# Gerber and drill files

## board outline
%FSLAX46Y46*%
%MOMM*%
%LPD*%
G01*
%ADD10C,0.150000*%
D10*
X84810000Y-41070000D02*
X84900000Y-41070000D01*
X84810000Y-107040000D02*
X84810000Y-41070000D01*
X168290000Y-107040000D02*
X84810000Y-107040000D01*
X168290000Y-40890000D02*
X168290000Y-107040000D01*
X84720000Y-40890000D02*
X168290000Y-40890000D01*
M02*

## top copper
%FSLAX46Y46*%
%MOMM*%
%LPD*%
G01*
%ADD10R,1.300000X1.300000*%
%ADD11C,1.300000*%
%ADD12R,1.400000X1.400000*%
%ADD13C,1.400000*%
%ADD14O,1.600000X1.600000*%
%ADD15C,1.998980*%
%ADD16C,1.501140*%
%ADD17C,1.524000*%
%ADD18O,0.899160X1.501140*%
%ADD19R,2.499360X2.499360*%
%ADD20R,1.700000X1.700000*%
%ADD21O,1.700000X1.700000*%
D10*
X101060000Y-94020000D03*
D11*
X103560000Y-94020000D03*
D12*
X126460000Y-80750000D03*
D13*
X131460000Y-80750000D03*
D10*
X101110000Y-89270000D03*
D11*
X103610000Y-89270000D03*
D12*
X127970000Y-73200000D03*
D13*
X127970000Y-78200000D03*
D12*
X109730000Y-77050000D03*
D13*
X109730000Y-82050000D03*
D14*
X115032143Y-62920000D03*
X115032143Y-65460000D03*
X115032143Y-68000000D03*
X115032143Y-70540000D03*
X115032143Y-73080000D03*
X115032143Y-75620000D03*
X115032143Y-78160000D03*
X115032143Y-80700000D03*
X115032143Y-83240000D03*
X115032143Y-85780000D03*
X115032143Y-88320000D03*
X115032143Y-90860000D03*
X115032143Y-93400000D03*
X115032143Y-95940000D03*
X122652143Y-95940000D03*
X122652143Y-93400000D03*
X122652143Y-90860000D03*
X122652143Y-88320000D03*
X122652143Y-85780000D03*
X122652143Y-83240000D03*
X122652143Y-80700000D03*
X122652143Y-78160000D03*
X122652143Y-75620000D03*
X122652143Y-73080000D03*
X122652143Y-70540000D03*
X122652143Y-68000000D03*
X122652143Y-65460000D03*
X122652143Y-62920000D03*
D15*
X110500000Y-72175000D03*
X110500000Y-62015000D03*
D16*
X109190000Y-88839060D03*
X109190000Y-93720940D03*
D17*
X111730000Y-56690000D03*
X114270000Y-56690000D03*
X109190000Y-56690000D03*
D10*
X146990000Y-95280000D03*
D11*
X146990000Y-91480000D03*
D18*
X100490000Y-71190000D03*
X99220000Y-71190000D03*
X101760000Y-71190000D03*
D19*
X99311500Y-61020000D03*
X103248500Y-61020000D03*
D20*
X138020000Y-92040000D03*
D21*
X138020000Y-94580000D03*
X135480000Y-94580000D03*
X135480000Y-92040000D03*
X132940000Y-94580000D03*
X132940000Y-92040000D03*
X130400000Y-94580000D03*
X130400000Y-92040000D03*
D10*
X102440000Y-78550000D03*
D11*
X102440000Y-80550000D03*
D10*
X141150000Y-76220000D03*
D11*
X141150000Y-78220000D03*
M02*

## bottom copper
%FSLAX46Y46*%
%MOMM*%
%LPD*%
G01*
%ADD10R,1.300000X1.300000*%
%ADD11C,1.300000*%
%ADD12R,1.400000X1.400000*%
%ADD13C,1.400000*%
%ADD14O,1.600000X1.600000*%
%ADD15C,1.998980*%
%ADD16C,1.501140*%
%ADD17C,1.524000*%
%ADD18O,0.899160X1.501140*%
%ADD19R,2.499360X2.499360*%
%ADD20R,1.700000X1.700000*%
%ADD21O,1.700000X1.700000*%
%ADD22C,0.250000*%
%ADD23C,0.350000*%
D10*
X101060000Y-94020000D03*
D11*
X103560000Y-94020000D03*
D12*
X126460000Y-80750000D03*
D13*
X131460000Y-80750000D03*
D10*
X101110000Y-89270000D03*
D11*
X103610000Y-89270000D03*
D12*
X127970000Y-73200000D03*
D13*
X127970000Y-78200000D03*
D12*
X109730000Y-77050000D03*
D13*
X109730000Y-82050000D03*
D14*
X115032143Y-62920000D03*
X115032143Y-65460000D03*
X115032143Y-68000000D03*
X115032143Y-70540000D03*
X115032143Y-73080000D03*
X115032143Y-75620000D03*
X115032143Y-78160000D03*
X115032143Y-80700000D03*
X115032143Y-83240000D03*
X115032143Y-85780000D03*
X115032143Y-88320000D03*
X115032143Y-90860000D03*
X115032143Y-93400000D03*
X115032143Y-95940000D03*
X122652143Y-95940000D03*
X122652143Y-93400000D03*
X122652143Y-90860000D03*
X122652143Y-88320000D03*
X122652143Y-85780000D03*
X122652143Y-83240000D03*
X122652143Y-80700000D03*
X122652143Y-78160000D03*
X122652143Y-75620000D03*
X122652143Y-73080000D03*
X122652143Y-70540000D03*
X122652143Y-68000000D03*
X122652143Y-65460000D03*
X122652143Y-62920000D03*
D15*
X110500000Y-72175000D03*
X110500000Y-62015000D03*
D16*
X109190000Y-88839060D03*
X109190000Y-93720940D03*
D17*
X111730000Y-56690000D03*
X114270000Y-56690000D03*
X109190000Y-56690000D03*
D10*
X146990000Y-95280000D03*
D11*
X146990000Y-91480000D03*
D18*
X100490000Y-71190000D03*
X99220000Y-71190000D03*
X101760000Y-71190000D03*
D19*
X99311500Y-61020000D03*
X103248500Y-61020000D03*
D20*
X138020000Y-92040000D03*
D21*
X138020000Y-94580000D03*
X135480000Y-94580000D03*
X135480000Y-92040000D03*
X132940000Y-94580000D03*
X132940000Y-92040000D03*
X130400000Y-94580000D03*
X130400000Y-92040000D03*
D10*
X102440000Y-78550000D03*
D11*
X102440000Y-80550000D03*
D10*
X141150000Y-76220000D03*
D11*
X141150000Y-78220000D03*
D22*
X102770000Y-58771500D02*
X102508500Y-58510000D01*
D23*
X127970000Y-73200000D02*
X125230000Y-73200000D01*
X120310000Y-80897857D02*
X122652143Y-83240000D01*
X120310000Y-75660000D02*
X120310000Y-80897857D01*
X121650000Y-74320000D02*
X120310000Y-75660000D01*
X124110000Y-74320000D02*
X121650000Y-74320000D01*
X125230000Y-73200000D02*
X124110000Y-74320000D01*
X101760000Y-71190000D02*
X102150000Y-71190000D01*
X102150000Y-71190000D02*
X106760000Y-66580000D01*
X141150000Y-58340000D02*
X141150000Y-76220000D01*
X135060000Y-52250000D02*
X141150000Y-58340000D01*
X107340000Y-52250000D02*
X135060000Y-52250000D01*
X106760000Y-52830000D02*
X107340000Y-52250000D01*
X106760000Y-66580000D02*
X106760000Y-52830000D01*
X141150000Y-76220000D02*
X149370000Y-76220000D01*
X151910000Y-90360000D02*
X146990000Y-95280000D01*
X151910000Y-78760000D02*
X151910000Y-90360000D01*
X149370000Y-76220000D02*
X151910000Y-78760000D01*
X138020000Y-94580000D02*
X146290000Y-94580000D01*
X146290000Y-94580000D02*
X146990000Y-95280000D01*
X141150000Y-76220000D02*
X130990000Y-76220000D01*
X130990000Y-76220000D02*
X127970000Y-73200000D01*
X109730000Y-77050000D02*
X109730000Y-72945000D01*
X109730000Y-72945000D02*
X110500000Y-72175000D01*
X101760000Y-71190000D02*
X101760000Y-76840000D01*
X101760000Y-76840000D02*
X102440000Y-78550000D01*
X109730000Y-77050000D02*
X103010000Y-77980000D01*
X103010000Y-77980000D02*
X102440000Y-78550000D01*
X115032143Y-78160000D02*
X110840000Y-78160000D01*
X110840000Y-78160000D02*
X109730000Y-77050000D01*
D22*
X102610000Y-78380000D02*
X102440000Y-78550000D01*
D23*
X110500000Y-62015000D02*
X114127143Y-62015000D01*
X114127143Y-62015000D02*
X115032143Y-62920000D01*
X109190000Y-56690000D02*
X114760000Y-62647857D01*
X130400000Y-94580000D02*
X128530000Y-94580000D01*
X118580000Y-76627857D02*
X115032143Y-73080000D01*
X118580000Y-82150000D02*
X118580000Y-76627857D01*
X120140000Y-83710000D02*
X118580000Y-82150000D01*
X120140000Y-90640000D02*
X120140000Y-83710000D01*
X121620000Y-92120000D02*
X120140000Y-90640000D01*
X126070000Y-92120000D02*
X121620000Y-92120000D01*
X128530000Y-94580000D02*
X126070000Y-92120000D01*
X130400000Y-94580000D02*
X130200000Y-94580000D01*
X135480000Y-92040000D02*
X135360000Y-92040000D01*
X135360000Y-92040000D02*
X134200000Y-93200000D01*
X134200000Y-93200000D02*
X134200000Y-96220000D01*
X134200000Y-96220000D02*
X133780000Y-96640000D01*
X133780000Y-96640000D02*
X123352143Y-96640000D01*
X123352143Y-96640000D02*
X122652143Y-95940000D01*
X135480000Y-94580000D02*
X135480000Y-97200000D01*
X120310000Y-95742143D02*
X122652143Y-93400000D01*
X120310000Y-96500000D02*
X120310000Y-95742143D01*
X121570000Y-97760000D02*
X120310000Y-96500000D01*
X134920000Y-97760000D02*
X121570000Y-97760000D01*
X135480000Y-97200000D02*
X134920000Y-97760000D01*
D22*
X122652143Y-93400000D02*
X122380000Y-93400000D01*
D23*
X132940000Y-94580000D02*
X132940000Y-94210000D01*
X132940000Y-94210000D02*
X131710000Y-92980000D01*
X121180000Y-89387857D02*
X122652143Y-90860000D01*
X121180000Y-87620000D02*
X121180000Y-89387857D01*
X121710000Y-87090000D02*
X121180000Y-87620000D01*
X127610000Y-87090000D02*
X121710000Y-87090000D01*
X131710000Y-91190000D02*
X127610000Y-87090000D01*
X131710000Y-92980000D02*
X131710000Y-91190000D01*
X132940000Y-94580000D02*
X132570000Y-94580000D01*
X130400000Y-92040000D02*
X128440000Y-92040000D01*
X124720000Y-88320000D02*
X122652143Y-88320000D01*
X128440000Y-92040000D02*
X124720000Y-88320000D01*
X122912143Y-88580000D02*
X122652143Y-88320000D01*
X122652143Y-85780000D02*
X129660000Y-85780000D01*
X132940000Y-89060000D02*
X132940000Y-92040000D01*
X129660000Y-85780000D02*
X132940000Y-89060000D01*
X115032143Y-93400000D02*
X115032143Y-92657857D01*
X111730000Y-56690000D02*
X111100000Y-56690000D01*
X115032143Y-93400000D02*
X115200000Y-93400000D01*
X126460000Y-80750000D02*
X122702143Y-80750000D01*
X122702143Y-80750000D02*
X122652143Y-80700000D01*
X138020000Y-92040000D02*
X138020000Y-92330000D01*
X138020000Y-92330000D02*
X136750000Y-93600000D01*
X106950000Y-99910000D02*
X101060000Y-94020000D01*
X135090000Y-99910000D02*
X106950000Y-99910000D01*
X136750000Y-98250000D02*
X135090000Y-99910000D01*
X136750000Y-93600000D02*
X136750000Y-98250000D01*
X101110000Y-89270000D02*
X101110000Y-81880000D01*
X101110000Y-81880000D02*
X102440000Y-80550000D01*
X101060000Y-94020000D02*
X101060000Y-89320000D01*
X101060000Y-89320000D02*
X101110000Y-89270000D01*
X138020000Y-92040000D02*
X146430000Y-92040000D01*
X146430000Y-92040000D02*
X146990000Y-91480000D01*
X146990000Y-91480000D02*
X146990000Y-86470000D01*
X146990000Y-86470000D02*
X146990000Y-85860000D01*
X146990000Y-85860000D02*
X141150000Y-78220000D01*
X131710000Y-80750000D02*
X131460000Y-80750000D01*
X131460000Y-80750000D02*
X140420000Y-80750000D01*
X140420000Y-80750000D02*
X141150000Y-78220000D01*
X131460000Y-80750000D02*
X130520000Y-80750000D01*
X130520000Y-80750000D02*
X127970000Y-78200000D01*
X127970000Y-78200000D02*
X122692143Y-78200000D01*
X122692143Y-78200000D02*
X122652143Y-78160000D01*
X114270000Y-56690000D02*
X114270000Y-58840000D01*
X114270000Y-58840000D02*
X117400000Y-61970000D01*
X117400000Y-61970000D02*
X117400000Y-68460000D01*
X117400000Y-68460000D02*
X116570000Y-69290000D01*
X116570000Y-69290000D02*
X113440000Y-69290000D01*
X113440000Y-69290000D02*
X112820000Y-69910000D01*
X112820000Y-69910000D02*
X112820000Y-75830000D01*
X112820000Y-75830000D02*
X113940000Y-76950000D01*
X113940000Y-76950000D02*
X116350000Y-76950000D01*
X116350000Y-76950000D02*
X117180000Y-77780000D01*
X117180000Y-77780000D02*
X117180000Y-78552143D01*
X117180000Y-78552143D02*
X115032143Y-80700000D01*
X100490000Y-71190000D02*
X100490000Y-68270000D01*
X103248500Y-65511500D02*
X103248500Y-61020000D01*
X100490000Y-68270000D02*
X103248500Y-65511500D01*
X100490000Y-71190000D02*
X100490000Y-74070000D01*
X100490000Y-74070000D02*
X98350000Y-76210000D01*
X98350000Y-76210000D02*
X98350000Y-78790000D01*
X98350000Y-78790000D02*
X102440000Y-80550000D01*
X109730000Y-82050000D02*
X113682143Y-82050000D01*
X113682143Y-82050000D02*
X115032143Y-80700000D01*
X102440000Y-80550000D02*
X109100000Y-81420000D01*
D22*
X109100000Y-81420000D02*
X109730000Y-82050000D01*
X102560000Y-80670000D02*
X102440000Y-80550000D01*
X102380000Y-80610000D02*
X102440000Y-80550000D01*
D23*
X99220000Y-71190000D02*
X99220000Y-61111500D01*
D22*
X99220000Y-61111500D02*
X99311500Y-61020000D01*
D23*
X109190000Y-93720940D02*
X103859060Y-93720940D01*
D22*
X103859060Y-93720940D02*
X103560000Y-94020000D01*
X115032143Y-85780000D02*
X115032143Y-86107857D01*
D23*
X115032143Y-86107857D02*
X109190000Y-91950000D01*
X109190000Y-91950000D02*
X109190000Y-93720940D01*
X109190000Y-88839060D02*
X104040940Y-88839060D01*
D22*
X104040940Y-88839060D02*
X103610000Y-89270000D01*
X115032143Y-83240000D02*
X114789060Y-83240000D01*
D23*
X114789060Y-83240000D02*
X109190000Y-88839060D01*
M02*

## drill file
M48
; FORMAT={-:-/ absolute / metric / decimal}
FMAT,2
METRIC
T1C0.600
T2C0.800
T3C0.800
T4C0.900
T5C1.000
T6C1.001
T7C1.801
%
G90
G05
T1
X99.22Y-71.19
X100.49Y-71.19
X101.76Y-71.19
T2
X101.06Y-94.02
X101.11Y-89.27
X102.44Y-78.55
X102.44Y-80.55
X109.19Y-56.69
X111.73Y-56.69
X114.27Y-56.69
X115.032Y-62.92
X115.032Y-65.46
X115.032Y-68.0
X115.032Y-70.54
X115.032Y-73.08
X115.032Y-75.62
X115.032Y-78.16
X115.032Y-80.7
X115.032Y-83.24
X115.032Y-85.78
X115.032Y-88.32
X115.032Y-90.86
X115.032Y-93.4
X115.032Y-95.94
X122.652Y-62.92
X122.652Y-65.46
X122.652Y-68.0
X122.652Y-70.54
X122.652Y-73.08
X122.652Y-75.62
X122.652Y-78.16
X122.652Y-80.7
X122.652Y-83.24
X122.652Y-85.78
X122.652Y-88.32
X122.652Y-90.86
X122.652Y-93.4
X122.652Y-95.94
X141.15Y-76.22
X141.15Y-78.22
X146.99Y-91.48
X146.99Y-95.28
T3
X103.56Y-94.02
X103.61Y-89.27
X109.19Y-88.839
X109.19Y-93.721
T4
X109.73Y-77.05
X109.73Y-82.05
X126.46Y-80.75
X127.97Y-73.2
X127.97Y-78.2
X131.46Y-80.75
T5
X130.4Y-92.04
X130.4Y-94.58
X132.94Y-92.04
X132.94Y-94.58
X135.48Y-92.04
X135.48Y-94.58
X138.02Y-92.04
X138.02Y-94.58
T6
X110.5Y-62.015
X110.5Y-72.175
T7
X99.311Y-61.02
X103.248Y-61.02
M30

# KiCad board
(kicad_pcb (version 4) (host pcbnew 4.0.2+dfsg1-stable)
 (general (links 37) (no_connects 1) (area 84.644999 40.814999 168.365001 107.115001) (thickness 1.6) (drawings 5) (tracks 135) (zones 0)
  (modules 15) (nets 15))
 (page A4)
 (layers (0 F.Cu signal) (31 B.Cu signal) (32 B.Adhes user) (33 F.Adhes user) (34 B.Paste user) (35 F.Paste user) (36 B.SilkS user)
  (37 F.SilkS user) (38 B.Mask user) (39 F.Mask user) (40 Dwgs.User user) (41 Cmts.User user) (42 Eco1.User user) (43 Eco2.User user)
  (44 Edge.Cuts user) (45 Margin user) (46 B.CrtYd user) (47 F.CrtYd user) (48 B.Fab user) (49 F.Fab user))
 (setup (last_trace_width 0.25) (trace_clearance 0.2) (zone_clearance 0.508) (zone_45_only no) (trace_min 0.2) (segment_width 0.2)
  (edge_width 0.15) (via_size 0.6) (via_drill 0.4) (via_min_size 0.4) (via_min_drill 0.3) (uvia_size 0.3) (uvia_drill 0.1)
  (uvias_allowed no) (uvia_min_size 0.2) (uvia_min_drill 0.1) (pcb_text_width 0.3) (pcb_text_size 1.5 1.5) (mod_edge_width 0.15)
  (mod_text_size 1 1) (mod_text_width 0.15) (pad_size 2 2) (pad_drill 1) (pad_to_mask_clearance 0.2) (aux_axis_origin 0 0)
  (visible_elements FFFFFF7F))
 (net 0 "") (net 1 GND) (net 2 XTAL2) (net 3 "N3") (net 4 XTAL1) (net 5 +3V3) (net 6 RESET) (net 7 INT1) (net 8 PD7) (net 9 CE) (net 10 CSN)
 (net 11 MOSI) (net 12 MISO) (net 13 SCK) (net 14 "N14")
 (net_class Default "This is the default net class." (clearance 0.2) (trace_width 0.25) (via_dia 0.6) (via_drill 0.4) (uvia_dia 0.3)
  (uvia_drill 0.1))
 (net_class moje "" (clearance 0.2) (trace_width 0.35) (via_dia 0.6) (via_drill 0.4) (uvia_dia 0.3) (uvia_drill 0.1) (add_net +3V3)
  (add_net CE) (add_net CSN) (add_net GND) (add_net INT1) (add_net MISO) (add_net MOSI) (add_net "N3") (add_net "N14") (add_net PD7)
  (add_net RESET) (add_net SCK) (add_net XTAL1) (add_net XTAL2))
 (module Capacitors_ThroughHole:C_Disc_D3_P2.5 (layer F.Cu) (at 101.06 94.02)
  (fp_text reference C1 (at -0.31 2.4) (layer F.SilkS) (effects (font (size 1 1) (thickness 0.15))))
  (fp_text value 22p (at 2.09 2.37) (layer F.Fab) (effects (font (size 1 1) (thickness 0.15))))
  (pad 1 thru_hole rect (at 0 0) (size 1.3 1.3) (drill 0.8) (layers *.Cu *.Mask F.SilkS) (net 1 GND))
  (pad 2 thru_hole circle (at 2.5 0) (size 1.3 1.3) (drill 0.8001) (layers *.Cu *.Mask F.SilkS) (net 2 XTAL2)))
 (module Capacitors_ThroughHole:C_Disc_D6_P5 (layer F.Cu) (at 126.46 80.75)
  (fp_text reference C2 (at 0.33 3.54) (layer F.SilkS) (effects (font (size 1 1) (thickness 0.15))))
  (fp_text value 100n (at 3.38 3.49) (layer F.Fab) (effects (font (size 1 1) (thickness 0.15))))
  (pad 1 thru_hole rect (at 0 0) (size 1.4 1.4) (drill 0.9) (layers *.Cu *.Mask F.SilkS) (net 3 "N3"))
  (pad 2 thru_hole circle (at 5 0) (size 1.4 1.4) (drill 0.9) (layers *.Cu *.Mask F.SilkS) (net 1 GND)))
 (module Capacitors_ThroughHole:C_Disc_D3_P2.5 (layer F.Cu) (at 101.11 89.27)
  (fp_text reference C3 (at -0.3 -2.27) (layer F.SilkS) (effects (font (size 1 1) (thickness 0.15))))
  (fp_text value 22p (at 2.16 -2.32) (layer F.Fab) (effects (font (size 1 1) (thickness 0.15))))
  (pad 1 thru_hole rect (at 0 0) (size 1.3 1.3) (drill 0.8) (layers *.Cu *.Mask F.SilkS) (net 1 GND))
  (pad 2 thru_hole circle (at 2.5 0) (size 1.3 1.3) (drill 0.8001) (layers *.Cu *.Mask F.SilkS) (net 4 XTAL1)))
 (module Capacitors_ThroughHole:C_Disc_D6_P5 (layer F.Cu) (at 127.97 73.2 270)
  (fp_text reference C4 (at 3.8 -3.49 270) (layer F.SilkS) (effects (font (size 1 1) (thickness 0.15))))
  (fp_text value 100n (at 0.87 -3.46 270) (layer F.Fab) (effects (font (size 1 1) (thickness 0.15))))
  (pad 1 thru_hole rect (at 0 0 270) (size 1.4 1.4) (drill 0.9) (layers *.Cu *.Mask F.SilkS) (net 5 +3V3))
  (pad 2 thru_hole circle (at 5 0 270) (size 1.4 1.4) (drill 0.9) (layers *.Cu *.Mask F.SilkS) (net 1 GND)))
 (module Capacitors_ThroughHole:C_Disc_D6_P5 (layer F.Cu) (at 109.73 77.05 270)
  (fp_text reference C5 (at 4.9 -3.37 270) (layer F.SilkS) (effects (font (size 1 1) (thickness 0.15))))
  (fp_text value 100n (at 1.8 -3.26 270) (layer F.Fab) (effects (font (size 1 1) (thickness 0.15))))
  (pad 1 thru_hole rect (at 0 0 270) (size 1.4 1.4) (drill 0.9) (layers *.Cu *.Mask F.SilkS) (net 5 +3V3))
  (pad 2 thru_hole circle (at 5 0 270) (size 1.4 1.4) (drill 0.9) (layers *.Cu *.Mask F.SilkS) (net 1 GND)))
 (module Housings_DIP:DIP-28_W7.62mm (layer F.Cu) (at 115.032143 62.92)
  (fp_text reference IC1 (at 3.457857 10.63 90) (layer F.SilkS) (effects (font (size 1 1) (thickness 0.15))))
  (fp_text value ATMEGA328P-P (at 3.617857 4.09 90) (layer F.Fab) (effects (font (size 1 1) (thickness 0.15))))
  (pad 1 thru_hole oval (at 0 0) (size 1.6 1.6) (drill 0.8) (layers *.Cu *.Mask F.SilkS) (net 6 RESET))
  (pad 2 thru_hole oval (at 0 2.54) (size 1.6 1.6) (drill 0.8) (layers *.Cu *.Mask F.SilkS))
  (pad 3 thru_hole oval (at 0 5.08) (size 1.6 1.6) (drill 0.8) (layers *.Cu *.Mask F.SilkS))
  (pad 4 thru_hole oval (at 0 7.62) (size 1.6 1.6) (drill 0.8) (layers *.Cu *.Mask F.SilkS))
  (pad 5 thru_hole oval (at 0 10.16) (size 1.6 1.6) (drill 0.8) (layers *.Cu *.Mask F.SilkS) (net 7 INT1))
  (pad 6 thru_hole oval (at 0 12.7) (size 1.6 1.6) (drill 0.8) (layers *.Cu *.Mask F.SilkS))
  (pad 7 thru_hole oval (at 0 15.24) (size 1.6 1.6) (drill 0.8) (layers *.Cu *.Mask F.SilkS) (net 5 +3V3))
  (pad 8 thru_hole oval (at 0 17.78) (size 1.6 1.6) (drill 0.8) (layers *.Cu *.Mask F.SilkS) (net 1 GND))
  (pad 9 thru_hole oval (at 0 20.32) (size 1.6 1.6) (drill 0.8) (layers *.Cu *.Mask F.SilkS) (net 4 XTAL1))
  (pad 10 thru_hole oval (at 0 22.86) (size 1.6 1.6) (drill 0.8) (layers *.Cu *.Mask F.SilkS) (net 2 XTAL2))
  (pad 11 thru_hole oval (at 0 25.4) (size 1.6 1.6) (drill 0.8) (layers *.Cu *.Mask F.SilkS))
  (pad 12 thru_hole oval (at 0 27.94) (size 1.6 1.6) (drill 0.8) (layers *.Cu *.Mask F.SilkS))
  (pad 13 thru_hole oval (at 0 30.48) (size 1.6 1.6) (drill 0.8) (layers *.Cu *.Mask F.SilkS) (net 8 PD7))
  (pad 14 thru_hole oval (at 0 33.02) (size 1.6 1.6) (drill 0.8) (layers *.Cu *.Mask F.SilkS))
  (pad 15 thru_hole oval (at 7.62 33.02) (size 1.6 1.6) (drill 0.8) (layers *.Cu *.Mask F.SilkS) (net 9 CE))
  (pad 16 thru_hole oval (at 7.62 30.48) (size 1.6 1.6) (drill 0.8) (layers *.Cu *.Mask F.SilkS) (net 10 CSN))
  (pad 17 thru_hole oval (at 7.62 27.94) (size 1.6 1.6) (drill 0.8) (layers *.Cu *.Mask F.SilkS) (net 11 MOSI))
  (pad 18 thru_hole oval (at 7.62 25.4) (size 1.6 1.6) (drill 0.8) (layers *.Cu *.Mask F.SilkS) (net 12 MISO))
  (pad 19 thru_hole oval (at 7.62 22.86) (size 1.6 1.6) (drill 0.8) (layers *.Cu *.Mask F.SilkS) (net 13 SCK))
  (pad 20 thru_hole oval (at 7.62 20.32) (size 1.6 1.6) (drill 0.8) (layers *.Cu *.Mask F.SilkS) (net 5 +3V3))
  (pad 21 thru_hole oval (at 7.62 17.78) (size 1.6 1.6) (drill 0.8) (layers *.Cu *.Mask F.SilkS) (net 3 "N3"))
  (pad 22 thru_hole oval (at 7.62 15.24) (size 1.6 1.6) (drill 0.8) (layers *.Cu *.Mask F.SilkS) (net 1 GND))
  (pad 23 thru_hole oval (at 7.62 12.7) (size 1.6 1.6) (drill 0.8) (layers *.Cu *.Mask F.SilkS))
  (pad 24 thru_hole oval (at 7.62 10.16) (size 1.6 1.6) (drill 0.8) (layers *.Cu *.Mask F.SilkS))
  (pad 25 thru_hole oval (at 7.62 7.62) (size 1.6 1.6) (drill 0.8) (layers *.Cu *.Mask F.SilkS))
  (pad 26 thru_hole oval (at 7.62 5.08) (size 1.6 1.6) (drill 0.8) (layers *.Cu *.Mask F.SilkS))
  (pad 27 thru_hole oval (at 7.62 2.54) (size 1.6 1.6) (drill 0.8) (layers *.Cu *.Mask F.SilkS))
  (pad 28 thru_hole oval (at 7.62 0) (size 1.6 1.6) (drill 0.8) (layers *.Cu *.Mask F.SilkS)))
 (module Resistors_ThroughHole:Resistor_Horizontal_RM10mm (layer F.Cu) (at 110.5 72.175 90)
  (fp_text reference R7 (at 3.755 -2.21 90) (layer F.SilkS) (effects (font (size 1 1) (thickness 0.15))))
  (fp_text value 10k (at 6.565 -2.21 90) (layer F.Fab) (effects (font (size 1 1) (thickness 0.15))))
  (pad 1 thru_hole circle (at 0 0 90) (size 1.99898 1.99898) (drill 1.00076) (layers *.Cu *.SilkS *.Mask) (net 5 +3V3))
  (pad 2 thru_hole circle (at 10.16 0 90) (size 1.99898 1.99898) (drill 1.00076) (layers *.Cu *.SilkS *.Mask) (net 6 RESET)))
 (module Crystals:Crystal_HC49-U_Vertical (layer F.Cu) (at 109.19 91.28 270)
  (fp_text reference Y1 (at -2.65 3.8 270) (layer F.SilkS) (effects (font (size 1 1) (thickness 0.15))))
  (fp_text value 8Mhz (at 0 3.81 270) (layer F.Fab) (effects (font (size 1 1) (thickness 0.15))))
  (pad 1 thru_hole circle (at -2.44094 0 270) (size 1.50114 1.50114) (drill 0.8001) (layers *.Cu *.Mask F.SilkS) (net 4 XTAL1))
  (pad 2 thru_hole circle (at 2.44094 0 270) (size 1.50114 1.50114) (drill 0.8001) (layers *.Cu *.Mask F.SilkS) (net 2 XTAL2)))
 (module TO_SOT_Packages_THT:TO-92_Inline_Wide (layer F.Cu) (at 109.19 56.69)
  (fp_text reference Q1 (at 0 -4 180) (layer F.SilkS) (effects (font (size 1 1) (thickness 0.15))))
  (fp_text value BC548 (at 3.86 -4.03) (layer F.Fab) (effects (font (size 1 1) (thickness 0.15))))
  (pad 2 thru_hole circle (at 2.54 0 90) (size 1.524 1.524) (drill 0.8) (layers *.Cu *.Mask F.SilkS) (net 8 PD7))
  (pad 3 thru_hole circle (at 5.08 0 90) (size 1.524 1.524) (drill 0.8) (layers *.Cu *.Mask F.SilkS) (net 1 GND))
  (pad 1 thru_hole circle (at 0 0 90) (size 1.524 1.524) (drill 0.8) (layers *.Cu *.Mask F.SilkS) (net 6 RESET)))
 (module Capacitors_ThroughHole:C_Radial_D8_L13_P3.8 (layer F.Cu) (at 146.99 95.28 90)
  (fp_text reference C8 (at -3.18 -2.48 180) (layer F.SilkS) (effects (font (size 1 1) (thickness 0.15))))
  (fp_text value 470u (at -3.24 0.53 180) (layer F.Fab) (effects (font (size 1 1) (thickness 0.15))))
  (pad 1 thru_hole rect (at 0 0 90) (size 1.3 1.3) (drill 0.8) (layers *.Cu *.Mask F.SilkS) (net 5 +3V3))
  (pad 2 thru_hole circle (at 3.8 0 90) (size 1.3 1.3) (drill 0.8) (layers *.Cu *.Mask F.SilkS) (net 1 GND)))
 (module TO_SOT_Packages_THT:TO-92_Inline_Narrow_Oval (layer F.Cu) (at 101.76 71.19 180)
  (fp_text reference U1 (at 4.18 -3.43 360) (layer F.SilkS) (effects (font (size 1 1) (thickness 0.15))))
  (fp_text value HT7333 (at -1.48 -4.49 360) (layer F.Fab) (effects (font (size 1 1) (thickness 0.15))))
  (pad 2 thru_hole oval (at 1.27 0) (size 0.89916 1.50114) (drill 0.6) (layers *.Cu *.Mask F.SilkS) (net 1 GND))
  (pad 3 thru_hole oval (at 2.54 0) (size 0.89916 1.50114) (drill 0.6) (layers *.Cu *.Mask F.SilkS) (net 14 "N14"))
  (pad 1 thru_hole oval (at 0 0) (size 0.89916 1.50114) (drill 0.6) (layers *.Cu *.Mask F.SilkS) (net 5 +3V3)))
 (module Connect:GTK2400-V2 (layer F.Cu) (at 101.28 61.02 180)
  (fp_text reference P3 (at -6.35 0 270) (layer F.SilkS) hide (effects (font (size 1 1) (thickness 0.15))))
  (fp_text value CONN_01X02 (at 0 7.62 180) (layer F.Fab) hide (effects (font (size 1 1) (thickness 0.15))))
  (pad 2 thru_hole rect (at 1.9685 0 180) (size 2.49936 2.49936) (drill 1.80086) (layers *.Cu *.Mask F.SilkS) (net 14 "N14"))
  (pad 1 thru_hole rect (at -1.9685 0 180) (size 2.49936 2.49936) (drill 1.80086) (layers *.Cu *.Mask F.SilkS) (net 1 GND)))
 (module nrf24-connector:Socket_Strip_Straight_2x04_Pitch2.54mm (layer F.Cu) (at 138.02 94.58 270)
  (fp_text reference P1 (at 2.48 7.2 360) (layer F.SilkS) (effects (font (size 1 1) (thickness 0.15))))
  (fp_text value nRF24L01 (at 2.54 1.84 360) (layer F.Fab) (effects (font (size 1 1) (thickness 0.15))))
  (pad 1 thru_hole rect (at -2.54 0 270) (size 1.7 1.7) (drill 1) (layers *.Cu *.Mask) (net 1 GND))
  (pad 2 thru_hole oval (at 0 0 270) (size 1.7 1.7) (drill 1) (layers *.Cu *.Mask) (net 5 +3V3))
  (pad 4 thru_hole oval (at 0 2.54 270) (size 1.7 1.7) (drill 1) (layers *.Cu *.Mask) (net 10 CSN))
  (pad 3 thru_hole oval (at -2.54 2.54 270) (size 1.7 1.7) (drill 1) (layers *.Cu *.Mask) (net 9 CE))
  (pad 6 thru_hole oval (at 0 5.08 270) (size 1.7 1.7) (drill 1) (layers *.Cu *.Mask) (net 11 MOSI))
  (pad 5 thru_hole oval (at -2.54 5.08 270) (size 1.7 1.7) (drill 1) (layers *.Cu *.Mask) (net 13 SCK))
  (pad 8 thru_hole oval (at 0 7.62 270) (size 1.7 1.7) (drill 1) (layers *.Cu *.Mask) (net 7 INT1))
  (pad 7 thru_hole oval (at -2.54 7.62 270) (size 1.7 1.7) (drill 1) (layers *.Cu *.Mask) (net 12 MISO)))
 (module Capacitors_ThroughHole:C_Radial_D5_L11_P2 (layer F.Cu) (at 102.44 78.55 270)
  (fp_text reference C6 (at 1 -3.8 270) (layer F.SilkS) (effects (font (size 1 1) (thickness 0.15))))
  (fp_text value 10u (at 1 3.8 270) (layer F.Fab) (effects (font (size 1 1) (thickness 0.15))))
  (pad 1 thru_hole rect (at 0 0 270) (size 1.3 1.3) (drill 0.8) (layers *.Cu *.Mask F.SilkS) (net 5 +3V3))
  (pad 2 thru_hole circle (at 2 0 270) (size 1.3 1.3) (drill 0.8) (layers *.Cu *.Mask F.SilkS) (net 1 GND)))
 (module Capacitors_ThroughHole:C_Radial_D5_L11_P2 (layer F.Cu) (at 141.15 76.22 270)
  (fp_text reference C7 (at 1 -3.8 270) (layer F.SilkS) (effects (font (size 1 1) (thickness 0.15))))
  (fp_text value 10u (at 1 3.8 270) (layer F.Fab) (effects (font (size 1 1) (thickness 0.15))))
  (pad 1 thru_hole rect (at 0 0 270) (size 1.3 1.3) (drill 0.8) (layers *.Cu *.Mask F.SilkS) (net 5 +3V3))
  (pad 2 thru_hole circle (at 2 0 270) (size 1.3 1.3) (drill 0.8) (layers *.Cu *.Mask F.SilkS) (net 1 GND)))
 (gr_line (start 84.81 41.07) (end 84.9 41.07) (angle 90) (layer Edge.Cuts) (width 0.15))
 (gr_line (start 84.81 107.04) (end 84.81 41.07) (angle 90) (layer Edge.Cuts) (width 0.15))
 (gr_line (start 168.29 107.04) (end 84.81 107.04) (angle 90) (layer Edge.Cuts) (width 0.15))
 (gr_line (start 168.29 40.89) (end 168.29 107.04) (angle 90) (layer Edge.Cuts) (width 0.15))
 (gr_line (start 84.72 40.89) (end 168.29 40.89) (angle 90) (layer Edge.Cuts) (width 0.15))
 (segment (start 102.77 58.7715) (end 102.5085 58.51) (width 0.25) (layer B.Cu) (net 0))
 (segment (start 127.97 73.2) (end 125.23 73.2) (width 0.35) (layer B.Cu) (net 5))
 (segment (start 120.31 80.897857) (end 122.652143 83.24) (width 0.35) (layer B.Cu) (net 5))
 (segment (start 120.31 75.66) (end 120.31 80.897857) (width 0.35) (layer B.Cu) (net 5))
 (segment (start 121.65 74.32) (end 120.31 75.66) (width 0.35) (layer B.Cu) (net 5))
 (segment (start 124.11 74.32) (end 121.65 74.32) (width 0.35) (layer B.Cu) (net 5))
 (segment (start 125.23 73.2) (end 124.11 74.32) (width 0.35) (layer B.Cu) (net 5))
 (segment (start 101.76 71.19) (end 102.15 71.19) (width 0.35) (layer B.Cu) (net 5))
 (segment (start 102.15 71.19) (end 106.76 66.58) (width 0.35) (layer B.Cu) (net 5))
 (segment (start 141.15 58.34) (end 141.15 76.22) (width 0.35) (layer B.Cu) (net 5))
 (segment (start 135.06 52.25) (end 141.15 58.34) (width 0.35) (layer B.Cu) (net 5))
 (segment (start 107.34 52.25) (end 135.06 52.25) (width 0.35) (layer B.Cu) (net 5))
 (segment (start 106.76 52.83) (end 107.34 52.25) (width 0.35) (layer B.Cu) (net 5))
 (segment (start 106.76 66.58) (end 106.76 52.83) (width 0.35) (layer B.Cu) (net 5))
 (segment (start 141.15 76.22) (end 149.37 76.22) (width 0.35) (layer B.Cu) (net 5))
 (segment (start 151.91 90.36) (end 146.99 95.28) (width 0.35) (layer B.Cu) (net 5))
 (segment (start 151.91 78.76) (end 151.91 90.36) (width 0.35) (layer B.Cu) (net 5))
 (segment (start 149.37 76.22) (end 151.91 78.76) (width 0.35) (layer B.Cu) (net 5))
 (segment (start 138.02 94.58) (end 146.29 94.58) (width 0.35) (layer B.Cu) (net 5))
 (segment (start 146.29 94.58) (end 146.99 95.28) (width 0.35) (layer B.Cu) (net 5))
 (segment (start 141.15 76.22) (end 130.99 76.22) (width 0.35) (layer B.Cu) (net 5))
 (segment (start 130.99 76.22) (end 127.97 73.2) (width 0.35) (layer B.Cu) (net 5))
 (segment (start 109.73 77.05) (end 109.73 72.945) (width 0.35) (layer B.Cu) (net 5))
 (segment (start 109.73 72.945) (end 110.5 72.175) (width 0.35) (layer B.Cu) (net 5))
 (segment (start 101.76 71.19) (end 101.76 76.84) (width 0.35) (layer B.Cu) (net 5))
 (segment (start 101.76 76.84) (end 102.44 78.55) (width 0.35) (layer B.Cu) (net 5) (status 20))
 (segment (start 109.73 77.05) (end 103.01 77.98) (width 0.35) (layer B.Cu) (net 5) (status 20))
 (segment (start 103.01 77.98) (end 102.44 78.55) (width 0.35) (layer B.Cu) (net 5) (status 30))
 (segment (start 115.032143 78.16) (end 110.84 78.16) (width 0.35) (layer B.Cu) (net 5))
 (segment (start 110.84 78.16) (end 109.73 77.05) (width 0.35) (layer B.Cu) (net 5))
 (segment (start 102.61 78.38) (end 102.44 78.55) (width 0.25) (layer B.Cu) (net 5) (status 30))
 (segment (start 110.5 62.015) (end 114.127143 62.015) (width 0.35) (layer B.Cu) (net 6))
 (segment (start 114.127143 62.015) (end 115.032143 62.92) (width 0.35) (layer B.Cu) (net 6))
 (segment (start 109.19 56.69) (end 114.76 62.647857) (width 0.35) (layer B.Cu) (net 6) (status 10))
 (segment (start 130.4 94.58) (end 128.53 94.58) (width 0.35) (layer B.Cu) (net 7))
 (segment (start 118.58 76.627857) (end 115.032143 73.08) (width 0.35) (layer B.Cu) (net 7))
 (segment (start 118.58 82.15) (end 118.58 76.627857) (width 0.35) (layer B.Cu) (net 7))
 (segment (start 120.14 83.71) (end 118.58 82.15) (width 0.35) (layer B.Cu) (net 7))
 (segment (start 120.14 90.64) (end 120.14 83.71) (width 0.35) (layer B.Cu) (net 7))
 (segment (start 121.62 92.12) (end 120.14 90.64) (width 0.35) (layer B.Cu) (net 7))
 (segment (start 126.07 92.12) (end 121.62 92.12) (width 0.35) (layer B.Cu) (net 7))
 (segment (start 128.53 94.58) (end 126.07 92.12) (width 0.35) (layer B.Cu) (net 7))
 (segment (start 130.4 94.58) (end 130.2 94.58) (width 0.35) (layer B.Cu) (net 7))
 (segment (start 135.48 92.04) (end 135.36 92.04) (width 0.35) (layer B.Cu) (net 9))
 (segment (start 135.36 92.04) (end 134.2 93.2) (width 0.35) (layer B.Cu) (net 9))
 (segment (start 134.2 93.2) (end 134.2 96.22) (width 0.35) (layer B.Cu) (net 9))
 (segment (start 134.2 96.22) (end 133.78 96.64) (width 0.35) (layer B.Cu) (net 9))
 (segment (start 133.78 96.64) (end 123.352143 96.64) (width 0.35) (layer B.Cu) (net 9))
 (segment (start 123.352143 96.64) (end 122.652143 95.94) (width 0.35) (layer B.Cu) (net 9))
 (segment (start 135.48 94.58) (end 135.48 97.2) (width 0.35) (layer B.Cu) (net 10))
 (segment (start 120.31 95.742143) (end 122.652143 93.4) (width 0.35) (layer B.Cu) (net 10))
 (segment (start 120.31 96.5) (end 120.31 95.742143) (width 0.35) (layer B.Cu) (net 10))
 (segment (start 121.57 97.76) (end 120.31 96.5) (width 0.35) (layer B.Cu) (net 10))
 (segment (start 134.92 97.76) (end 121.57 97.76) (width 0.35) (layer B.Cu) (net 10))
 (segment (start 135.48 97.2) (end 134.92 97.76) (width 0.35) (layer B.Cu) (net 10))
 (segment (start 122.652143 93.4) (end 122.38 93.4) (width 0.25) (layer B.Cu) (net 10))
 (segment (start 132.94 94.58) (end 132.94 94.21) (width 0.35) (layer B.Cu) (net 11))
 (segment (start 132.94 94.21) (end 131.71 92.98) (width 0.35) (layer B.Cu) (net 11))
 (segment (start 121.18 89.387857) (end 122.652143 90.86) (width 0.35) (layer B.Cu) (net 11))
 (segment (start 121.18 87.62) (end 121.18 89.387857) (width 0.35) (layer B.Cu) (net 11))
 (segment (start 121.71 87.09) (end 121.18 87.62) (width 0.35) (layer B.Cu) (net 11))
 (segment (start 127.61 87.09) (end 121.71 87.09) (width 0.35) (layer B.Cu) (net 11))
 (segment (start 131.71 91.19) (end 127.61 87.09) (width 0.35) (layer B.Cu) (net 11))
 (segment (start 131.71 92.98) (end 131.71 91.19) (width 0.35) (layer B.Cu) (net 11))
 (segment (start 132.94 94.58) (end 132.57 94.58) (width 0.35) (layer B.Cu) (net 11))
 (segment (start 130.4 92.04) (end 128.44 92.04) (width 0.35) (layer B.Cu) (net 12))
 (segment (start 124.72 88.32) (end 122.652143 88.32) (width 0.35) (layer B.Cu) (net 12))
 (segment (start 128.44 92.04) (end 124.72 88.32) (width 0.35) (layer B.Cu) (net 12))
 (segment (start 122.912143 88.58) (end 122.652143 88.32) (width 0.35) (layer B.Cu) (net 12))
 (segment (start 122.652143 85.78) (end 129.66 85.78) (width 0.35) (layer B.Cu) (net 13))
 (segment (start 132.94 89.06) (end 132.94 92.04) (width 0.35) (layer B.Cu) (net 13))
 (segment (start 129.66 85.78) (end 132.94 89.06) (width 0.35) (layer B.Cu) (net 13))
 (segment (start 115.032143 93.4) (end 115.032143 92.657857) (width 0.35) (layer B.Cu) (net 8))
 (segment (start 111.73 56.69) (end 111.1 56.69) (width 0.35) (layer B.Cu) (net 8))
 (segment (start 115.032143 93.4) (end 115.2 93.4) (width 0.35) (layer B.Cu) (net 8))
 (segment (start 126.46 80.75) (end 122.702143 80.75) (width 0.35) (layer B.Cu) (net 3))
 (segment (start 122.702143 80.75) (end 122.652143 80.7) (width 0.35) (layer B.Cu) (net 3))
 (segment (start 138.02 92.04) (end 138.02 92.33) (width 0.35) (layer B.Cu) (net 1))
 (segment (start 138.02 92.33) (end 136.75 93.6) (width 0.35) (layer B.Cu) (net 1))
 (segment (start 106.95 99.91) (end 101.06 94.02) (width 0.35) (layer B.Cu) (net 1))
 (segment (start 135.09 99.91) (end 106.95 99.91) (width 0.35) (layer B.Cu) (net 1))
 (segment (start 136.75 98.25) (end 135.09 99.91) (width 0.35) (layer B.Cu) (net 1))
 (segment (start 136.75 93.6) (end 136.75 98.25) (width 0.35) (layer B.Cu) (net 1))
 (segment (start 101.11 89.27) (end 101.11 81.88) (width 0.35) (layer B.Cu) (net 1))
 (segment (start 101.11 81.88) (end 102.44 80.55) (width 0.35) (layer B.Cu) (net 1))
 (segment (start 101.06 94.02) (end 101.06 89.32) (width 0.35) (layer B.Cu) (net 1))
 (segment (start 101.06 89.32) (end 101.11 89.27) (width 0.35) (layer B.Cu) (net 1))
 (segment (start 138.02 92.04) (end 146.43 92.04) (width 0.35) (layer B.Cu) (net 1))
 (segment (start 146.43 92.04) (end 146.99 91.48) (width 0.35) (layer B.Cu) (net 1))
 (segment (start 146.99 91.48) (end 146.99 86.47) (width 0.35) (layer B.Cu) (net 1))
 (segment (start 146.99 86.47) (end 146.99 85.86) (width 0.35) (layer B.Cu) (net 1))
 (segment (start 146.99 85.86) (end 141.15 78.22) (width 0.35) (layer B.Cu) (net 1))
 (segment (start 131.71 80.75) (end 131.46 80.75) (width 0.35) (layer B.Cu) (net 1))
 (segment (start 131.46 80.75) (end 140.42 80.75) (width 0.35) (layer B.Cu) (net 1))
 (segment (start 140.42 80.75) (end 141.15 78.22) (width 0.35) (layer B.Cu) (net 1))
 (segment (start 131.46 80.75) (end 130.52 80.75) (width 0.35) (layer B.Cu) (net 1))
 (segment (start 130.52 80.75) (end 127.97 78.2) (width 0.35) (layer B.Cu) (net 1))
 (segment (start 127.97 78.2) (end 122.692143 78.2) (width 0.35) (layer B.Cu) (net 1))
 (segment (start 122.692143 78.2) (end 122.652143 78.16) (width 0.35) (layer B.Cu) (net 1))
 (segment (start 114.27 56.69) (end 114.27 58.84) (width 0.35) (layer B.Cu) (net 1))
 (segment (start 114.27 58.84) (end 117.4 61.97) (width 0.35) (layer B.Cu) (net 1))
 (segment (start 117.4 61.97) (end 117.4 68.46) (width 0.35) (layer B.Cu) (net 1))
 (segment (start 117.4 68.46) (end 116.57 69.29) (width 0.35) (layer B.Cu) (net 1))
 (segment (start 116.57 69.29) (end 113.44 69.29) (width 0.35) (layer B.Cu) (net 1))
 (segment (start 113.44 69.29) (end 112.82 69.91) (width 0.35) (layer B.Cu) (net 1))
 (segment (start 112.82 69.91) (end 112.82 75.83) (width 0.35) (layer B.Cu) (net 1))
 (segment (start 112.82 75.83) (end 113.94 76.95) (width 0.35) (layer B.Cu) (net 1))
 (segment (start 113.94 76.95) (end 116.35 76.95) (width 0.35) (layer B.Cu) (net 1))
 (segment (start 116.35 76.95) (end 117.18 77.78) (width 0.35) (layer B.Cu) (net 1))
 (segment (start 117.18 77.78) (end 117.18 78.552143) (width 0.35) (layer B.Cu) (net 1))
 (segment (start 117.18 78.552143) (end 115.032143 80.7) (width 0.35) (layer B.Cu) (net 1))
 (segment (start 100.49 71.19) (end 100.49 68.27) (width 0.35) (layer B.Cu) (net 1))
 (segment (start 103.2485 65.5115) (end 103.2485 61.02) (width 0.35) (layer B.Cu) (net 1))
 (segment (start 100.49 68.27) (end 103.2485 65.5115) (width 0.35) (layer B.Cu) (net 1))
 (segment (start 100.49 71.19) (end 100.49 74.07) (width 0.35) (layer B.Cu) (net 1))
 (segment (start 100.49 74.07) (end 98.35 76.21) (width 0.35) (layer B.Cu) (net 1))
 (segment (start 98.35 76.21) (end 98.35 78.79) (width 0.35) (layer B.Cu) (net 1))
 (segment (start 98.35 78.79) (end 102.44 80.55) (width 0.35) (layer B.Cu) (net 1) (status 20))
 (segment (start 109.73 82.05) (end 113.682143 82.05) (width 0.35) (layer B.Cu) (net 1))
 (segment (start 113.682143 82.05) (end 115.032143 80.7) (width 0.35) (layer B.Cu) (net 1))
 (segment (start 102.44 80.55) (end 109.1 81.42) (width 0.35) (layer B.Cu) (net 1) (status 10))
 (segment (start 109.1 81.42) (end 109.73 82.05) (width 0.25) (layer B.Cu) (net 1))
 (segment (start 102.56 80.67) (end 102.44 80.55) (width 0.25) (layer B.Cu) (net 1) (status 30))
 (segment (start 102.38 80.61) (end 102.44 80.55) (width 0.25) (layer B.Cu) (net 1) (status 30))
 (segment (start 99.22 71.19) (end 99.22 61.1115) (width 0.35) (layer B.Cu) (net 14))
 (segment (start 99.22 61.1115) (end 99.3115 61.02) (width 0.25) (layer B.Cu) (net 14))
 (segment (start 109.19 93.72094) (end 103.85906 93.72094) (width 0.35) (layer B.Cu) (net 2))
 (segment (start 103.85906 93.72094) (end 103.56 94.02) (width 0.25) (layer B.Cu) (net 2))
 (segment (start 115.032143 85.78) (end 115.032143 86.107857) (width 0.25) (layer B.Cu) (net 2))
 (segment (start 115.032143 86.107857) (end 109.19 91.95) (width 0.35) (layer B.Cu) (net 2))
 (segment (start 109.19 91.95) (end 109.19 93.72094) (width 0.35) (layer B.Cu) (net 2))
 (segment (start 109.19 88.83906) (end 104.04094 88.83906) (width 0.35) (layer B.Cu) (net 4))
 (segment (start 104.04094 88.83906) (end 103.61 89.27) (width 0.25) (layer B.Cu) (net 4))
 (segment (start 115.032143 83.24) (end 114.78906 83.24) (width 0.25) (layer B.Cu) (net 4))
 (segment (start 114.78906 83.24) (end 109.19 88.83906) (width 0.35) (layer B.Cu) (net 4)))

